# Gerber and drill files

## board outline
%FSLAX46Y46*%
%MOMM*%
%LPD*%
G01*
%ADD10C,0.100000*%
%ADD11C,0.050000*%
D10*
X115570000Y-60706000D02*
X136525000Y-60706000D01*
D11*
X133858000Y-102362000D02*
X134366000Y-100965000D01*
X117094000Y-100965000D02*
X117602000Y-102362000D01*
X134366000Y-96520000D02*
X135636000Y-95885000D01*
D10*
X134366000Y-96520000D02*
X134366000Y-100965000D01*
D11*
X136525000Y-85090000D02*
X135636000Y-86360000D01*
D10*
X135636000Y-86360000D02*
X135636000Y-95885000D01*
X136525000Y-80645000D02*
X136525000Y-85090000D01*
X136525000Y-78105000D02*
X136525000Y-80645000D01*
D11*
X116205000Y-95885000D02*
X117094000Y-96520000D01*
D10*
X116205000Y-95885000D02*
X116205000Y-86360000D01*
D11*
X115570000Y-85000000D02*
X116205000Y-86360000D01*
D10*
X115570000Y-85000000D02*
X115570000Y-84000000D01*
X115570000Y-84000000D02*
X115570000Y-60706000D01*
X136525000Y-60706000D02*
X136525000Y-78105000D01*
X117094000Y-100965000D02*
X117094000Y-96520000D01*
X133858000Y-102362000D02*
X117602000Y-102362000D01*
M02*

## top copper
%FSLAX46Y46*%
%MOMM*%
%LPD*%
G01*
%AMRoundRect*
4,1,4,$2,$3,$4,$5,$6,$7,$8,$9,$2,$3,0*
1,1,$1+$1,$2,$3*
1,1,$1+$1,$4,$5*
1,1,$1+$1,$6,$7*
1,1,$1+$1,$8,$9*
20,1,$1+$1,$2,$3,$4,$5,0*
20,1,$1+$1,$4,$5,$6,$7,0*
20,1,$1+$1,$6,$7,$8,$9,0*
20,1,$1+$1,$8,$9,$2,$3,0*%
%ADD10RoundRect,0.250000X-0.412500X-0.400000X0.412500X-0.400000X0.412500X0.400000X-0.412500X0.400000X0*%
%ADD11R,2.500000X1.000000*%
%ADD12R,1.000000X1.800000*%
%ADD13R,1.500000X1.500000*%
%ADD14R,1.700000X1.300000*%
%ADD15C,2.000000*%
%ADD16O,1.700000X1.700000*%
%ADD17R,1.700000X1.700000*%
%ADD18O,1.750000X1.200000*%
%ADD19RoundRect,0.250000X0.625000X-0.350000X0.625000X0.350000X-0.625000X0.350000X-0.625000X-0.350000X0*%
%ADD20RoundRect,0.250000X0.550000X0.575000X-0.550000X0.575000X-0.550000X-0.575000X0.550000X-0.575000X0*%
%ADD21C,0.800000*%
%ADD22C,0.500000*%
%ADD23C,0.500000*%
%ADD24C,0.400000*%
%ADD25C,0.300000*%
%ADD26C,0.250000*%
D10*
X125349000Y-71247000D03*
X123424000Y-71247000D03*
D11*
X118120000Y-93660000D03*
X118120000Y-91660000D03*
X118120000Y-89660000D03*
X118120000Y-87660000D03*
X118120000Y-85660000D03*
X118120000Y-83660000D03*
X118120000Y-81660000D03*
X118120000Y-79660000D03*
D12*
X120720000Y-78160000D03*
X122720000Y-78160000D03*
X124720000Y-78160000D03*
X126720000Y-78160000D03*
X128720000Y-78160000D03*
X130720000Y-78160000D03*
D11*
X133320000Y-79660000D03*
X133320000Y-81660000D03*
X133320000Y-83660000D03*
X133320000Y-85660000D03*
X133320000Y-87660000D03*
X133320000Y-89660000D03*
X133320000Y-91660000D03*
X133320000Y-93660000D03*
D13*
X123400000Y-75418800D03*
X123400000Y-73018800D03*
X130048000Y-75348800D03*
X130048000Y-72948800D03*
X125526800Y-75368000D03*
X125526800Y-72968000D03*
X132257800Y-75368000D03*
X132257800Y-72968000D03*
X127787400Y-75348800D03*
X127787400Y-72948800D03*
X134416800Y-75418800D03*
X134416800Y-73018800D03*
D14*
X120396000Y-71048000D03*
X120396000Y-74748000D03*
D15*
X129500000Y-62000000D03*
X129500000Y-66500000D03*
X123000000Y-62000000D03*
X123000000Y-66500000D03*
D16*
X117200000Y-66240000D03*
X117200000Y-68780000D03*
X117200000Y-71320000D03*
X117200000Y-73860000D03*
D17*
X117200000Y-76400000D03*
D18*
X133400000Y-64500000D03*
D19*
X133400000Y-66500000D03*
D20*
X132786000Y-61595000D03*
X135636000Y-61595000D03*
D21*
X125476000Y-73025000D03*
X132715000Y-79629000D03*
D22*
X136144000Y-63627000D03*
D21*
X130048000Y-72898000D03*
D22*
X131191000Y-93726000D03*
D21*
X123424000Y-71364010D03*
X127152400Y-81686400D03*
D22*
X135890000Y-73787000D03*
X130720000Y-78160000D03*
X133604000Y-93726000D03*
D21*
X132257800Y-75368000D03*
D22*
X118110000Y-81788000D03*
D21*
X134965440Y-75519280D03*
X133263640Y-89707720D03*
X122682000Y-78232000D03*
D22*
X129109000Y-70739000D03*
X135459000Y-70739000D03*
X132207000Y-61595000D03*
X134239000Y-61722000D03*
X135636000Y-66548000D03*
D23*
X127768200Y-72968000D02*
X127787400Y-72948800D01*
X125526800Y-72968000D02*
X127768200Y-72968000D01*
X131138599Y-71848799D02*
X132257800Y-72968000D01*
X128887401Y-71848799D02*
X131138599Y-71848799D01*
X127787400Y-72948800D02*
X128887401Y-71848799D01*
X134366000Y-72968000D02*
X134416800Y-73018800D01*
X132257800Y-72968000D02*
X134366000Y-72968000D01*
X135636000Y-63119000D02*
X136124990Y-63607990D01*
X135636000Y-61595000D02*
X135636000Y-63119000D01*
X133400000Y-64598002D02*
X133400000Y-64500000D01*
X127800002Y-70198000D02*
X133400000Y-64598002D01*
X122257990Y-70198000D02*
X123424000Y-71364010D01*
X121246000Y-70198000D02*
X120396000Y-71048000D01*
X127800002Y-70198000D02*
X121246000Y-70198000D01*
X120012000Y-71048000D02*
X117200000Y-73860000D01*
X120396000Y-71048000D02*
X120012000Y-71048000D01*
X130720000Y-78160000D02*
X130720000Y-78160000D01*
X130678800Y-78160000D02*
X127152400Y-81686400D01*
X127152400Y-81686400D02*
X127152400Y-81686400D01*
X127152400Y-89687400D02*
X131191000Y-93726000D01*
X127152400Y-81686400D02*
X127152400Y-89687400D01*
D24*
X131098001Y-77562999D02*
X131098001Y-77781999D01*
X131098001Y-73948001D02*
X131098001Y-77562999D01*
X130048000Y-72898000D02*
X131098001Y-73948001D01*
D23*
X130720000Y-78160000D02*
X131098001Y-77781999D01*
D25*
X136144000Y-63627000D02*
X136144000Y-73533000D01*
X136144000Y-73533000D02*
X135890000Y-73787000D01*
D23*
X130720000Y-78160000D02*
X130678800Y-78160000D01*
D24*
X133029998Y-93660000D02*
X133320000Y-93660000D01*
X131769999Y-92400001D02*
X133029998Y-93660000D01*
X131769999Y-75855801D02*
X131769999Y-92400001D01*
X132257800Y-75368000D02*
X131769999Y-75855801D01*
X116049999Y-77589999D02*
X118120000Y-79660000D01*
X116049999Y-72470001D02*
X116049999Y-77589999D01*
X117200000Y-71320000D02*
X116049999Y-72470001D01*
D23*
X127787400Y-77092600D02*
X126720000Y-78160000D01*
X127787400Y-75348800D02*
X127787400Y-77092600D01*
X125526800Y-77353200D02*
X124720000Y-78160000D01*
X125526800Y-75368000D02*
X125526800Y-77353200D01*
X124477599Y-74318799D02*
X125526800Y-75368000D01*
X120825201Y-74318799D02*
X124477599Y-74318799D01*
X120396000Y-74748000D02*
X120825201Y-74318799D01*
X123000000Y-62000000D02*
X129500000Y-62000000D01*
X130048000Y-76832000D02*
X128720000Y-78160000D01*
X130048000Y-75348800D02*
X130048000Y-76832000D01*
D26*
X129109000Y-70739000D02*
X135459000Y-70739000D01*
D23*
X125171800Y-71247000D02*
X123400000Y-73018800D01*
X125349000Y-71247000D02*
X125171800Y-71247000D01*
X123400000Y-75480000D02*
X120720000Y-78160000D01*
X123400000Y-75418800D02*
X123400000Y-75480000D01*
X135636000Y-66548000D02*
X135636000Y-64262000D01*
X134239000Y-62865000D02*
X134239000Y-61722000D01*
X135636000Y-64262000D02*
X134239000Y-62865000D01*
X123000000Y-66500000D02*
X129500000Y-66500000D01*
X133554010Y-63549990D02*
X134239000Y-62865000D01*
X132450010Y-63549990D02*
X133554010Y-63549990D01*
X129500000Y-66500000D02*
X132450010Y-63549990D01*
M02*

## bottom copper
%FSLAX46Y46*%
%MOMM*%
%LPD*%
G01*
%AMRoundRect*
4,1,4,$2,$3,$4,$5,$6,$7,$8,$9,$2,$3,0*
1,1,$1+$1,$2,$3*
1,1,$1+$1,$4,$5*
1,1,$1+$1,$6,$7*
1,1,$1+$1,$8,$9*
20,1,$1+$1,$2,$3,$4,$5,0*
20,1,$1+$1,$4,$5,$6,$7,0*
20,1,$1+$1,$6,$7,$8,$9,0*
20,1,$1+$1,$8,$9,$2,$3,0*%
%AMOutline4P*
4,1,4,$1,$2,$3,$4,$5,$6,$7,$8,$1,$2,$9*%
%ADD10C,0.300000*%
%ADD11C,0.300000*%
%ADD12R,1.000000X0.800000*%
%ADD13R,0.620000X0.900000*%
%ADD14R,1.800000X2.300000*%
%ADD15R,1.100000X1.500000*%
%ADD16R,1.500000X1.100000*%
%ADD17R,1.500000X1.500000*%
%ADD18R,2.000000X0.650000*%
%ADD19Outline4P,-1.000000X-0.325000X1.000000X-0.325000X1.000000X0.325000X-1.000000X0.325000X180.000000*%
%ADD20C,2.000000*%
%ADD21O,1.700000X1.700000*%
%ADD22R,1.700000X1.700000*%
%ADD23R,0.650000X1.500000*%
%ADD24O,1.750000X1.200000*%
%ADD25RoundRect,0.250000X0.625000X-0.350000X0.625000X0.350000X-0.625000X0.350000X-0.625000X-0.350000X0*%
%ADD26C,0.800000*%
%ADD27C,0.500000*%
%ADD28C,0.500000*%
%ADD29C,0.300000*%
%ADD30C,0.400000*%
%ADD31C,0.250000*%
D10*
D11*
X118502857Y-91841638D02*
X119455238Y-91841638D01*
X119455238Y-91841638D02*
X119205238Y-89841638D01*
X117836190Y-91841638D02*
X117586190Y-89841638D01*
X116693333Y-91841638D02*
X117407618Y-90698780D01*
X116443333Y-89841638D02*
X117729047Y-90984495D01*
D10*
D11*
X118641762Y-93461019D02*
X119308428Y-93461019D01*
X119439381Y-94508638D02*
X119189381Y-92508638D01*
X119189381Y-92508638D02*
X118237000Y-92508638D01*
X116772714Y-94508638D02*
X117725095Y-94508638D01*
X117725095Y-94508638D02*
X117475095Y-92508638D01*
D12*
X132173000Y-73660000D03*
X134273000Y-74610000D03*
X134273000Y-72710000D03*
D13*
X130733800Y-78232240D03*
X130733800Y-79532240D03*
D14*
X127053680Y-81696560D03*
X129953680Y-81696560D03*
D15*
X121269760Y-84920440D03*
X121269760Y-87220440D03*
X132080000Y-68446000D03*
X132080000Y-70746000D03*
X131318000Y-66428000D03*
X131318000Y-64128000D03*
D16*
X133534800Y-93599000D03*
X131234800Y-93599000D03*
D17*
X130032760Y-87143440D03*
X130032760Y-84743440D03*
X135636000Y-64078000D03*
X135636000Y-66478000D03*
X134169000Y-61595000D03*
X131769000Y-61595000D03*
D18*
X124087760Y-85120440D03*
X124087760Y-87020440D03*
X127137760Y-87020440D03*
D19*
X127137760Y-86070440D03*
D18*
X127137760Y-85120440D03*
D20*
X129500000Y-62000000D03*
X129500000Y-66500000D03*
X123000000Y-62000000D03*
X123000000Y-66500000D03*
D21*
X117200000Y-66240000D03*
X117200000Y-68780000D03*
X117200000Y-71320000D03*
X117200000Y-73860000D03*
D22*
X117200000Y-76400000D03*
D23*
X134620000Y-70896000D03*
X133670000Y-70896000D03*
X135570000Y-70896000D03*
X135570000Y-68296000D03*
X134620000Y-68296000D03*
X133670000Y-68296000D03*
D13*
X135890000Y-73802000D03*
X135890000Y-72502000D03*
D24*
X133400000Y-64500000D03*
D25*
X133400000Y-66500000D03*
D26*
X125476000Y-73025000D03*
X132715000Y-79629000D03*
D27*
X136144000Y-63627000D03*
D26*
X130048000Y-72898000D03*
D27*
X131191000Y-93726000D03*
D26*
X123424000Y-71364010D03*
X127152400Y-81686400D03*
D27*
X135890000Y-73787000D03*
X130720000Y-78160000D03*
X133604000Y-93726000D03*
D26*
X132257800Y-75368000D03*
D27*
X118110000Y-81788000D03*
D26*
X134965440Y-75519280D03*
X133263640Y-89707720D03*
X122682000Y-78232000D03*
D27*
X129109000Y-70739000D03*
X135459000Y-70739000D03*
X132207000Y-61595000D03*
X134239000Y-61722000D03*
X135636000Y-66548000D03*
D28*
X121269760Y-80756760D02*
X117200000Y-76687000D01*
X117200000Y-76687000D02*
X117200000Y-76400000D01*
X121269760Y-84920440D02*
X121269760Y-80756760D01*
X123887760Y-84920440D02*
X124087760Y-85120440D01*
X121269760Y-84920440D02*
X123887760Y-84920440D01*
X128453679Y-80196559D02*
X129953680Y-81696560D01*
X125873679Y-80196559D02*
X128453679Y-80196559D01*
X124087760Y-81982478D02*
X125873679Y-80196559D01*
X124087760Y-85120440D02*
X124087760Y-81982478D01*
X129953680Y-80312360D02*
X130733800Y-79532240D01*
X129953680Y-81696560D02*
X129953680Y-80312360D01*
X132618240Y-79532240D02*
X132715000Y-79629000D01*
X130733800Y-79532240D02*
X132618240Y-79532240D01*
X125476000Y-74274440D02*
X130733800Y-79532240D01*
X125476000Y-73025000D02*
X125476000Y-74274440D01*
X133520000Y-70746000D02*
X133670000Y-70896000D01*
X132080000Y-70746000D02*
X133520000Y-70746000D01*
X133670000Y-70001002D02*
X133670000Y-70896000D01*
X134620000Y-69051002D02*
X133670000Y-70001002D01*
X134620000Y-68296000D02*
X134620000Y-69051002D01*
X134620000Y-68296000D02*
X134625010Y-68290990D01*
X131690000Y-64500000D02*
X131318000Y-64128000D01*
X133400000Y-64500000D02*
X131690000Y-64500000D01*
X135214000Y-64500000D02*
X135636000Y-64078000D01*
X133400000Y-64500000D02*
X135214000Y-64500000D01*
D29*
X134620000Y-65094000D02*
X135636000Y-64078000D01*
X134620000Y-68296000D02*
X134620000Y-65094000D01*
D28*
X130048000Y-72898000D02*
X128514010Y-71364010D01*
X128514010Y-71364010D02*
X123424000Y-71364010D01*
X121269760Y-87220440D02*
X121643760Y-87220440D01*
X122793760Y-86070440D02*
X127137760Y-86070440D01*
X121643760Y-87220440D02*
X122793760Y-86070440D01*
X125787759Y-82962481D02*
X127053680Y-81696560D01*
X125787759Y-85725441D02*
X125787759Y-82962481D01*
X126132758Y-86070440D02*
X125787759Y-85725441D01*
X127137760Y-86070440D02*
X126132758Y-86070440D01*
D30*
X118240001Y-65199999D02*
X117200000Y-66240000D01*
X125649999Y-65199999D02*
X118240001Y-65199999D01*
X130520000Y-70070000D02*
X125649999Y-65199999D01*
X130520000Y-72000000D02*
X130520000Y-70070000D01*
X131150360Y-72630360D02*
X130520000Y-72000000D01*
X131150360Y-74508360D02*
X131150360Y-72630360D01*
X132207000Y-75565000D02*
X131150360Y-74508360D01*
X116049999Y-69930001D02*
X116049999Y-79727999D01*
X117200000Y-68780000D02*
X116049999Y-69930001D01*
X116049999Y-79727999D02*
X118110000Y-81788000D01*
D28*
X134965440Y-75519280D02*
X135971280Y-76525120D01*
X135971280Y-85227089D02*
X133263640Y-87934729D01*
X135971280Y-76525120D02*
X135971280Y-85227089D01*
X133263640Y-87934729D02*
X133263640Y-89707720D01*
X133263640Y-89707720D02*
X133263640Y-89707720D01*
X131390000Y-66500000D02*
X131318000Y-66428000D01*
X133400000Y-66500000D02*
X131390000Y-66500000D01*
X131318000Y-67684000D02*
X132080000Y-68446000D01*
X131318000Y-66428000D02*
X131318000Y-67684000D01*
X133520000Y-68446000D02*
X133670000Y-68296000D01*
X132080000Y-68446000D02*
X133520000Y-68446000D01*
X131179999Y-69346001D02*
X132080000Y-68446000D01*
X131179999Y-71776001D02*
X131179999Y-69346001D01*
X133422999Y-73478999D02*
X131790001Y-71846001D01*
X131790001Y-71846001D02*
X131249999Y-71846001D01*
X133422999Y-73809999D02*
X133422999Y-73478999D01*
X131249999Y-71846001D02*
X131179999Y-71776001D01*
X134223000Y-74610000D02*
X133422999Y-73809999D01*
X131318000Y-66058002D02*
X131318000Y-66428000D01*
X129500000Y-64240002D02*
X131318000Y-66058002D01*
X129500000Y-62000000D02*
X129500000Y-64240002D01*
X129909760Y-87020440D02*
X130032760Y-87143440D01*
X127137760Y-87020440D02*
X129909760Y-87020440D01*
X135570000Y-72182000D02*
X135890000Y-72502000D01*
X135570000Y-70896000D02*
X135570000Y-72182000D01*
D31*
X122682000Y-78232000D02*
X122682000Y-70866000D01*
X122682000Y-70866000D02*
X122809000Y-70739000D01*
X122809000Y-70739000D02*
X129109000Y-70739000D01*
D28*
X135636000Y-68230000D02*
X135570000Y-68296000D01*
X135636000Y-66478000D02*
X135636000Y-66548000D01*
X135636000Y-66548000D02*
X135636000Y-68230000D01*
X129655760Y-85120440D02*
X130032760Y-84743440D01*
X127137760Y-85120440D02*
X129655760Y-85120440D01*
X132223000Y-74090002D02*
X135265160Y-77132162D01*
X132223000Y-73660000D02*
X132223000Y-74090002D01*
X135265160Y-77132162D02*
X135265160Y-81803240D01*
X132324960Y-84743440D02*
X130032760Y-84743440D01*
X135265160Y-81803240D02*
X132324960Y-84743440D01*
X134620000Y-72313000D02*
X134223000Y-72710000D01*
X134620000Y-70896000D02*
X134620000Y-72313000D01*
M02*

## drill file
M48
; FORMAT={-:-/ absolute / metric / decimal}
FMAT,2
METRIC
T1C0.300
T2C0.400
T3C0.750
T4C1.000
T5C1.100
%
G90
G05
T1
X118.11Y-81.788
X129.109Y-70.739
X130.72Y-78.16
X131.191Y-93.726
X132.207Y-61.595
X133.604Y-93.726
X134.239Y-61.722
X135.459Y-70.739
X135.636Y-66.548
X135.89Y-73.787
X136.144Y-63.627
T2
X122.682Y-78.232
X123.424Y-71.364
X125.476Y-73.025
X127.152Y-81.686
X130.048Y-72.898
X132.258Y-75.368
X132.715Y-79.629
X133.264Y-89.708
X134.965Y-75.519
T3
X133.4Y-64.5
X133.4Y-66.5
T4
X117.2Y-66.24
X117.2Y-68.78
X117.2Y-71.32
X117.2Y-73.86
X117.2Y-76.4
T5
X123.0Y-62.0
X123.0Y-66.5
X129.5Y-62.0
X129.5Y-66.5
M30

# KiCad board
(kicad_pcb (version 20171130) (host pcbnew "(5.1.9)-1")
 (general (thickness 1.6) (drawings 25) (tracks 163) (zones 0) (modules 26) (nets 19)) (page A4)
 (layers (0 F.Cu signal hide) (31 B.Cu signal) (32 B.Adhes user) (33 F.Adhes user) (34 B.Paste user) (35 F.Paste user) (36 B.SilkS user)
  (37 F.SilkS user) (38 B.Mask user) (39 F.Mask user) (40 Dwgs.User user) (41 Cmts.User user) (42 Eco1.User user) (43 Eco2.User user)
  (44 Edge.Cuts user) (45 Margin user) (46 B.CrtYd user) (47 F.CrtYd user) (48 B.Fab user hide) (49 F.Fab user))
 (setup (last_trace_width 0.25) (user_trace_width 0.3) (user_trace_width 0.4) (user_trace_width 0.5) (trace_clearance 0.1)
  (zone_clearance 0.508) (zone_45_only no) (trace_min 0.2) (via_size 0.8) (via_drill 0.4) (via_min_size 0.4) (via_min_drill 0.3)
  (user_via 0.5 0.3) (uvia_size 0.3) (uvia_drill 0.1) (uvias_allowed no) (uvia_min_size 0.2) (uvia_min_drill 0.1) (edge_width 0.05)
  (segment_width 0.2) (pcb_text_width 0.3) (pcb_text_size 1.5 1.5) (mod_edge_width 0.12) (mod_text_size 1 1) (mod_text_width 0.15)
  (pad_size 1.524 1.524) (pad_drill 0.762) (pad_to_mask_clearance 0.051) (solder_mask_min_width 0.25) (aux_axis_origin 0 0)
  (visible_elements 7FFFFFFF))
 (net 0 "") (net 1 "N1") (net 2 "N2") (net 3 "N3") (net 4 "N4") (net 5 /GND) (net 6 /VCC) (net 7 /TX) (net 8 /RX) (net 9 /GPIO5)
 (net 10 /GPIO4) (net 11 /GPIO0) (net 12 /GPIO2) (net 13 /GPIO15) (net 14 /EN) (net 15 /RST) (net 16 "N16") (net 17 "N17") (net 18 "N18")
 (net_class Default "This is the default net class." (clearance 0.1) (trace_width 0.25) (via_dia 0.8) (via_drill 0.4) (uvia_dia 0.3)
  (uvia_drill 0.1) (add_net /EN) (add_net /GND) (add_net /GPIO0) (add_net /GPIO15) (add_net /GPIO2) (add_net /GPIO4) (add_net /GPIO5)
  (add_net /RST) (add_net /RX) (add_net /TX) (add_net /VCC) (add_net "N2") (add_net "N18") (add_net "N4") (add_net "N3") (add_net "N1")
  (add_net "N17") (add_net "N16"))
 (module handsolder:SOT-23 (layer B.Cu) (at 133.223 73.66 180)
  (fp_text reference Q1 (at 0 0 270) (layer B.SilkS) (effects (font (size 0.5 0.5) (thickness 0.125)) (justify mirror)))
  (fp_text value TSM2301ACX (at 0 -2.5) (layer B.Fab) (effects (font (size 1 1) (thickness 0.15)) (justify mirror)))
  (pad 3 smd rect (at 1.05 0 180) (size 1 0.8) (layers B.Cu B.Paste B.Mask) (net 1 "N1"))
  (pad 2 smd rect (at -1.05 -0.95 180) (size 1 0.8) (layers B.Cu B.Paste B.Mask) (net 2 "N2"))
  (pad 1 smd rect (at -1.05 0.95 180) (size 1 0.8) (layers B.Cu B.Paste B.Mask) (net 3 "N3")))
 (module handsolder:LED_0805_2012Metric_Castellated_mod (layer F.Cu) (at 124.3865 71.247)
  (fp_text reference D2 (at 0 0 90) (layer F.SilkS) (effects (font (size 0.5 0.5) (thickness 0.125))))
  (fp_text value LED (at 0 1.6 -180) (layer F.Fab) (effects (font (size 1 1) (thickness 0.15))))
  (pad 2 smd roundrect (at 0.9625 0) (size 1.325 1.3) (layers F.Cu F.Paste F.Mask) (roundrect_rratio 0.1923076923076923) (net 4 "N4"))
  (pad 1 smd roundrect (at -0.9625 0) (size 1.325 1.3) (layers F.Cu F.Paste F.Mask) (roundrect_rratio 0.1923076923076923) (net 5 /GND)))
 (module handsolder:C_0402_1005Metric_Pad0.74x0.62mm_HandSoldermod (layer B.Cu) (at 130.7338 78.88224 90)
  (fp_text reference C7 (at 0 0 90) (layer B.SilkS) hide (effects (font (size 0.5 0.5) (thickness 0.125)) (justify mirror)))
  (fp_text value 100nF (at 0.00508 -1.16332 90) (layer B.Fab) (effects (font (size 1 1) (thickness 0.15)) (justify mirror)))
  (pad 2 smd rect (at 0.65 0 90) (size 0.9 0.62) (layers B.Cu B.Paste B.Mask) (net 5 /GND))
  (pad 1 smd rect (at -0.65 0 90) (size 0.9 0.62) (layers B.Cu B.Paste B.Mask) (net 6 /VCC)))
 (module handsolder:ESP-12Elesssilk (layer F.Cu) (at 125.72 90.16 180)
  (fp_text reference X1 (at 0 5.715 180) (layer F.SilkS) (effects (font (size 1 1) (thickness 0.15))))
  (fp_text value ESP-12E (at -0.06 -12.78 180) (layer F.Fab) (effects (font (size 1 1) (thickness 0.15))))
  (pad 22 smd rect (at 7.6 -3.5 180) (size 2.5 1) (layers F.Cu F.Paste F.Mask))
  (pad 21 smd rect (at 7.6 -1.5 180) (size 2.5 1) (layers F.Cu F.Paste F.Mask))
  (pad 20 smd rect (at 7.6 0.5 180) (size 2.5 1) (layers F.Cu F.Paste F.Mask))
  (pad 19 smd rect (at 7.6 2.5 180) (size 2.5 1) (layers F.Cu F.Paste F.Mask))
  (pad 18 smd rect (at 7.6 4.5 180) (size 2.5 1) (layers F.Cu F.Paste F.Mask))
  (pad 17 smd rect (at 7.6 6.5 180) (size 2.5 1) (layers F.Cu F.Paste F.Mask))
  (pad 16 smd rect (at 7.6 8.5 180) (size 2.5 1) (layers F.Cu F.Paste F.Mask) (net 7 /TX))
  (pad 15 smd rect (at 7.6 10.5 180) (size 2.5 1) (layers F.Cu F.Paste F.Mask) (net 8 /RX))
  (pad 14 smd rect (at 5 12 180) (size 1 1.8) (layers F.Cu F.Paste F.Mask) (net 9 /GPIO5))
  (pad 13 smd rect (at 3 12 180) (size 1 1.8) (layers F.Cu F.Paste F.Mask) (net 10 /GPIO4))
  (pad 12 smd rect (at 1 12 180) (size 1 1.8) (layers F.Cu F.Paste F.Mask) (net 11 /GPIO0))
  (pad 11 smd rect (at -1 12 180) (size 1 1.8) (layers F.Cu F.Paste F.Mask) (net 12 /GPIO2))
  (pad 10 smd rect (at -3 12 180) (size 1 1.8) (layers F.Cu F.Paste F.Mask) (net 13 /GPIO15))
  (pad 9 smd rect (at -5 12 180) (size 1 1.8) (layers F.Cu F.Paste F.Mask) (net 5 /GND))
  (pad 8 smd rect (at -7.6 10.5 180) (size 2.5 1) (layers F.Cu F.Paste F.Mask) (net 6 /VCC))
  (pad 7 smd rect (at -7.6 8.5 180) (size 2.5 1) (layers F.Cu F.Paste F.Mask))
  (pad 6 smd rect (at -7.6 6.5 180) (size 2.5 1) (layers F.Cu F.Paste F.Mask))
  (pad 5 smd rect (at -7.6 4.5 180) (size 2.5 1) (layers F.Cu F.Paste F.Mask))
  (pad 4 smd rect (at -7.6 2.5 180) (size 2.5 1) (layers F.Cu F.Paste F.Mask))
  (pad 3 smd rect (at -7.6 0.5 180) (size 2.5 1) (layers F.Cu F.Paste F.Mask) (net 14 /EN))
  (pad 2 smd rect (at -7.6 -1.5 180) (size 2.5 1) (layers F.Cu F.Paste F.Mask))
  (pad 1 smd rect (at -7.6 -3.5 180) (size 2.5 1) (layers F.Cu F.Paste F.Mask) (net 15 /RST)))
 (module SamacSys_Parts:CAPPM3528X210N (layer B.Cu) (at 128.50368 81.69656 180)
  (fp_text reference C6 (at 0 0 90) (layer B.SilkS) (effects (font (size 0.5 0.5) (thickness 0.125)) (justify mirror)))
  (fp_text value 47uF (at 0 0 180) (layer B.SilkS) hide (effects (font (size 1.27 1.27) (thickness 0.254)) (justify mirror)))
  (pad 2 smd rect (at 1.45 0 180) (size 1.8 2.3) (layers B.Cu B.Paste B.Mask) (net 5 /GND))
  (pad 1 smd rect (at -1.45 0 180) (size 1.8 2.3) (layers B.Cu B.Paste B.Mask) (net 6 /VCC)))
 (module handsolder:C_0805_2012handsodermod (layer B.Cu) (at 121.26976 86.07044 90)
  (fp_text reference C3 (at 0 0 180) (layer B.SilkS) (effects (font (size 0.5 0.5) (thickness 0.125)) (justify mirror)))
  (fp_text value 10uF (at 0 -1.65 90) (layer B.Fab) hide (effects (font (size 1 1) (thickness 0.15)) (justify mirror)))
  (pad 2 smd rect (at 1.15 0 90) (size 1.5 1.1) (layers B.Cu B.Paste B.Mask) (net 6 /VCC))
  (pad 1 smd rect (at -1.15 0 90) (size 1.5 1.1) (layers B.Cu B.Paste B.Mask) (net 5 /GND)))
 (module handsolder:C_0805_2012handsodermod (layer B.Cu) (at 132.08 69.596 90)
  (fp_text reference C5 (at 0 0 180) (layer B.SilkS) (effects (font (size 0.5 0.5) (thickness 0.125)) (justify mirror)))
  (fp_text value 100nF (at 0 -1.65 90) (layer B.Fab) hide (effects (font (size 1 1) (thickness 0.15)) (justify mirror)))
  (pad 2 smd rect (at 1.15 0 90) (size 1.5 1.1) (layers B.Cu B.Paste B.Mask) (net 2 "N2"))
  (pad 1 smd rect (at -1.15 0 90) (size 1.5 1.1) (layers B.Cu B.Paste B.Mask) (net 5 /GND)))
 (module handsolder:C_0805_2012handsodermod (layer B.Cu) (at 131.318 65.278 270)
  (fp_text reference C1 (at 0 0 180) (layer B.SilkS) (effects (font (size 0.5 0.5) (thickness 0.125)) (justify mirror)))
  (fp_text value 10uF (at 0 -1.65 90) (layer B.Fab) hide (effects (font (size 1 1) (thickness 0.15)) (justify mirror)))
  (pad 2 smd rect (at 1.15 0 270) (size 1.5 1.1) (layers B.Cu B.Paste B.Mask) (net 2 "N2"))
  (pad 1 smd rect (at -1.15 0 270) (size 1.5 1.1) (layers B.Cu B.Paste B.Mask) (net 5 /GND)))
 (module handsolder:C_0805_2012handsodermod (layer B.Cu) (at 132.3848 93.599)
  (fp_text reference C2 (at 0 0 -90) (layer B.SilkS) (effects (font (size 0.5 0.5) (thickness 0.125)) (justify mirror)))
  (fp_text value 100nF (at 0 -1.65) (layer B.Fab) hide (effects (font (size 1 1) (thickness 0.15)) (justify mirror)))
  (pad 2 smd rect (at 1.15 0) (size 1.5 1.1) (layers B.Cu B.Paste B.Mask) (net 15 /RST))
  (pad 1 smd rect (at -1.15 0) (size 1.5 1.1) (layers B.Cu B.Paste B.Mask) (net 5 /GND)))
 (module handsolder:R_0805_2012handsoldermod (layer F.Cu) (at 123.4 74.2188 270)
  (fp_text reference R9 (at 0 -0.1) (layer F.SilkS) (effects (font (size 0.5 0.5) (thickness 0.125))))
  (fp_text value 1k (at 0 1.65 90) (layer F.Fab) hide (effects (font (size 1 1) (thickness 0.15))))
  (pad 2 smd rect (at 1.2 0 270) (size 1.5 1.5) (layers F.Cu F.Paste F.Mask) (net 9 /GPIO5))
  (pad 1 smd rect (at -1.2 0 270) (size 1.5 1.5) (layers F.Cu F.Paste F.Mask) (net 4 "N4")))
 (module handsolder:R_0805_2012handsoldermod (layer B.Cu) (at 130.03276 85.94344 270)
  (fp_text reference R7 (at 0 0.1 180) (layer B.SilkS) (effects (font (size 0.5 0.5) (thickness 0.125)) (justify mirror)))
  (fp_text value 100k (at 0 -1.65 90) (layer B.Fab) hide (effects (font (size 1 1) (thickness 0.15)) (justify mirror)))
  (pad 2 smd rect (at 1.2 0 270) (size 1.5 1.5) (layers B.Cu B.Paste B.Mask) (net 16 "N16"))
  (pad 1 smd rect (at -1.2 0 270) (size 1.5 1.5) (layers B.Cu B.Paste B.Mask) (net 1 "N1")))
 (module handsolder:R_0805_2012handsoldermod (layer B.Cu) (at 135.636 65.278 90)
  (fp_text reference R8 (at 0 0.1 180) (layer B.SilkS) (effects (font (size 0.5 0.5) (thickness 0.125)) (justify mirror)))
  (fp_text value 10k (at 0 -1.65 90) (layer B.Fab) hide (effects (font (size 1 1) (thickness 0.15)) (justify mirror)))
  (pad 2 smd rect (at 1.2 0 90) (size 1.5 1.5) (layers B.Cu B.Paste B.Mask) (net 5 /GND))
  (pad 1 smd rect (at -1.2 0 90) (size 1.5 1.5) (layers B.Cu B.Paste B.Mask) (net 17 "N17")))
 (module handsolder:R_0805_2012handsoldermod (layer B.Cu) (at 132.969 61.595)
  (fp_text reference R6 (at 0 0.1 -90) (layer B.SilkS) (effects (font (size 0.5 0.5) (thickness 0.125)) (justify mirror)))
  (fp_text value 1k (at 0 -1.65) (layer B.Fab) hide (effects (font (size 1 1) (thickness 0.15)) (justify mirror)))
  (pad 2 smd rect (at 1.2 0) (size 1.5 1.5) (layers B.Cu B.Paste B.Mask) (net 17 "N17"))
  (pad 1 smd rect (at -1.2 0) (size 1.5 1.5) (layers B.Cu B.Paste B.Mask) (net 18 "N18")))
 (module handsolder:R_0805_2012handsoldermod (layer F.Cu) (at 130.048 74.1488 270)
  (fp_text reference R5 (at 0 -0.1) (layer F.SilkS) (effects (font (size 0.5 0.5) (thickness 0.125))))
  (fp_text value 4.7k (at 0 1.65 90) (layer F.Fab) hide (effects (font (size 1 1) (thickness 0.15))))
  (pad 2 smd rect (at 1.2 0 270) (size 1.5 1.5) (layers F.Cu F.Paste F.Mask) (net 13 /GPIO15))
  (pad 1 smd rect (at -1.2 0 270) (size 1.5 1.5) (layers F.Cu F.Paste F.Mask) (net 5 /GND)))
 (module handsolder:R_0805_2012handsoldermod (layer F.Cu) (at 125.5268 74.168 270)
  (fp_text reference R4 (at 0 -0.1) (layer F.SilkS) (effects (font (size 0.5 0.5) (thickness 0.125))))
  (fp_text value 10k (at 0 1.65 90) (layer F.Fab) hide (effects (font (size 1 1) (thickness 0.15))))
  (pad 2 smd rect (at 1.2 0 270) (size 1.5 1.5) (layers F.Cu F.Paste F.Mask) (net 11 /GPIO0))
  (pad 1 smd rect (at -1.2 0 270) (size 1.5 1.5) (layers F.Cu F.Paste F.Mask) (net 6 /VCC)))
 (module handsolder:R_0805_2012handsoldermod (layer F.Cu) (at 132.2578 74.168 270)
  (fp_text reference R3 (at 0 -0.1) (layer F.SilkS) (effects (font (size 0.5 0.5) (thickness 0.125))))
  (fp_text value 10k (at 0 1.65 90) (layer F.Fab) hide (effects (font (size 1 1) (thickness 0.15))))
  (pad 2 smd rect (at 1.2 0 270) (size 1.5 1.5) (layers F.Cu F.Paste F.Mask) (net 15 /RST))
  (pad 1 smd rect (at -1.2 0 270) (size 1.5 1.5) (layers F.Cu F.Paste F.Mask) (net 6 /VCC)))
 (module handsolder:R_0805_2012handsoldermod (layer F.Cu) (at 127.7874 74.1488 270)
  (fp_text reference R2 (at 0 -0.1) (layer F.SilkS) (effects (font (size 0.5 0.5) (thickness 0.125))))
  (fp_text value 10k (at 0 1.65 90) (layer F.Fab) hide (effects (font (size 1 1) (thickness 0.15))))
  (pad 2 smd rect (at 1.2 0 270) (size 1.5 1.5) (layers F.Cu F.Paste F.Mask) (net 12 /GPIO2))
  (pad 1 smd rect (at -1.2 0 270) (size 1.5 1.5) (layers F.Cu F.Paste F.Mask) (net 6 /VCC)))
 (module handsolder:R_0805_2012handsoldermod (layer F.Cu) (at 134.4168 74.2188 270)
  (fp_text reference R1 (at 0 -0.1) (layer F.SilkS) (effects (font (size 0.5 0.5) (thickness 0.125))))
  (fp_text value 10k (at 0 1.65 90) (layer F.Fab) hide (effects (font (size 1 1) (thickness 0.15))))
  (pad 2 smd rect (at 1.2 0 270) (size 1.5 1.5) (layers F.Cu F.Paste F.Mask) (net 14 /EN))
  (pad 1 smd rect (at -1.2 0 270) (size 1.5 1.5) (layers F.Cu F.Paste F.Mask) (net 6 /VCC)))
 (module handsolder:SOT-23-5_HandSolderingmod (layer B.Cu) (at 125.58776 86.07044 180)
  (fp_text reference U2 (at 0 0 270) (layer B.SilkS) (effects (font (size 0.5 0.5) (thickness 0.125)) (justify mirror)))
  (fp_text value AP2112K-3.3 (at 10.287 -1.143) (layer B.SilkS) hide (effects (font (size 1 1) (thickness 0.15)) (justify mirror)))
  (pad 5 smd rect (at 1.5 0.95 180) (size 2 0.65) (layers B.Cu B.Paste B.Mask) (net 6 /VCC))
  (pad 4 smd rect (at 1.5 -0.95 180) (size 2 0.65) (layers B.Cu B.Paste B.Mask))
  (pad 3 smd rect (at -1.55 -0.95 180) (size 2 0.65) (layers B.Cu B.Paste B.Mask) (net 16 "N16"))
  (pad 2 smd trapezoid (at -1.55 0 180) (size 2 0.65) (layers B.Cu B.Paste B.Mask) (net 5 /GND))
  (pad 1 smd rect (at -1.55 0.95 180) (size 2 0.65) (layers B.Cu B.Paste B.Mask) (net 1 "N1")))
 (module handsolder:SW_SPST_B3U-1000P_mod (layer F.Cu) (at 120.396 72.898 90)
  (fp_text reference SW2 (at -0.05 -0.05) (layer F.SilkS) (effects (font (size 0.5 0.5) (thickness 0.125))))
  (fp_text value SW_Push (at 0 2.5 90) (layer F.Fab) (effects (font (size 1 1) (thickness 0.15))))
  (pad 2 smd rect (at 1.85 0 90) (size 1.3 1.7) (layers F.Cu F.Paste F.Mask) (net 5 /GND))
  (pad 1 smd rect (at -1.85 0 90) (size 1.3 1.7) (layers F.Cu F.Paste F.Mask) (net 11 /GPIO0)))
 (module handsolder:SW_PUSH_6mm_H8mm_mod (layer F.Cu) (at 123 62)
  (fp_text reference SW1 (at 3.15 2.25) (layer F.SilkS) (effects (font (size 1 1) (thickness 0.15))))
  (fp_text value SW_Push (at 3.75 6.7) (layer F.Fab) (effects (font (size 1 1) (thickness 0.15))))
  (pad 1 thru_hole circle (at 6.5 0 90) (size 2 2) (drill 1.1) (layers *.Cu *.Mask) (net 2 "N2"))
  (pad 2 thru_hole circle (at 6.5 4.5 90) (size 2 2) (drill 1.1) (layers *.Cu *.Mask) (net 17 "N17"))
  (pad 1 thru_hole circle (at 0 0 90) (size 2 2) (drill 1.1) (layers *.Cu *.Mask) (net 2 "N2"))
  (pad 2 thru_hole circle (at 0 4.5 90) (size 2 2) (drill 1.1) (layers *.Cu *.Mask) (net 17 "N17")))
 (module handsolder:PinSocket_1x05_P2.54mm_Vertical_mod (layer F.Cu) (at 117.2 76.4 180)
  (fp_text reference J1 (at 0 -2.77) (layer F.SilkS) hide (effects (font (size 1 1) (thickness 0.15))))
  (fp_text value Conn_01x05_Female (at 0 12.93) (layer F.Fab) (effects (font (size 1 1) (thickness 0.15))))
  (pad 5 thru_hole oval (at 0 10.16 180) (size 1.7 1.7) (drill 1) (layers *.Cu *.Mask) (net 15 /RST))
  (pad 4 thru_hole oval (at 0 7.62 180) (size 1.7 1.7) (drill 1) (layers *.Cu *.Mask) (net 7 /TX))
  (pad 3 thru_hole oval (at 0 5.08 180) (size 1.7 1.7) (drill 1) (layers *.Cu *.Mask) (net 8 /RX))
  (pad 2 thru_hole oval (at 0 2.54 180) (size 1.7 1.7) (drill 1) (layers *.Cu *.Mask) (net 5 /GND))
  (pad 1 thru_hole rect (at 0 0 180) (size 1.7 1.7) (drill 1) (layers *.Cu *.Mask) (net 6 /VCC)))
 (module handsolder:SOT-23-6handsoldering (layer B.Cu) (at 134.62 69.596 270)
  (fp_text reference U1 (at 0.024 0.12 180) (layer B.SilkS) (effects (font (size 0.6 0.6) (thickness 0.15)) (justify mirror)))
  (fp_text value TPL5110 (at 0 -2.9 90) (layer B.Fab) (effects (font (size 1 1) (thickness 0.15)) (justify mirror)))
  (pad 5 smd rect (at 1.3 0 270) (size 1.5 0.65) (layers B.Cu B.Paste B.Mask) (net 3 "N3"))
  (pad 6 smd rect (at 1.3 0.95 270) (size 1.5 0.65) (layers B.Cu B.Paste B.Mask) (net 5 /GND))
  (pad 4 smd rect (at 1.3 -0.95 270) (size 1.5 0.65) (layers B.Cu B.Paste B.Mask) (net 10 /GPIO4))
  (pad 3 smd rect (at -1.3 -0.95 270) (size 1.5 0.65) (layers B.Cu B.Paste B.Mask) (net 17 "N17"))
  (pad 2 smd rect (at -1.3 0 270) (size 1.5 0.65) (layers B.Cu B.Paste B.Mask) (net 5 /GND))
  (pad 1 smd rect (at -1.3 0.95 270) (size 1.5 0.65) (layers B.Cu B.Paste B.Mask) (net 2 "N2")))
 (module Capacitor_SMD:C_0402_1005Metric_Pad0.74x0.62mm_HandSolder (layer B.Cu) (at 135.89 73.152 270)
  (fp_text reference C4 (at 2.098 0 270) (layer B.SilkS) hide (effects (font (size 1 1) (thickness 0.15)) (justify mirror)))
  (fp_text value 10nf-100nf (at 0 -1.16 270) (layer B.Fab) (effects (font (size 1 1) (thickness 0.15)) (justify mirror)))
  (pad 2 smd rect (at 0.65 0 270) (size 0.9 0.62) (layers B.Cu B.Paste B.Mask) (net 5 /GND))
  (pad 1 smd rect (at -0.65 0 270) (size 0.9 0.62) (layers B.Cu B.Paste B.Mask) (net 10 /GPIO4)))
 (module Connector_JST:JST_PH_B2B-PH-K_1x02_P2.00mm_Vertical (layer F.Cu) (at 133.4 66.5 90)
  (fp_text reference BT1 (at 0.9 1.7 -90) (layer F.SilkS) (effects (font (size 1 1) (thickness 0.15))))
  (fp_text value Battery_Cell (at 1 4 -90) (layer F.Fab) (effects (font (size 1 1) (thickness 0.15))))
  (pad 2 thru_hole oval (at 2 0 90) (size 1.2 1.75) (drill 0.75) (layers *.Cu *.Mask) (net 5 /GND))
  (pad 1 thru_hole roundrect (at 0 0 90) (size 1.2 1.75) (drill 0.75) (layers *.Cu *.Mask) (roundrect_rratio 0.208333) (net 2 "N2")))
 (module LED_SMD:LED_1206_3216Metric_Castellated (layer F.Cu) (at 134.211 61.595 180)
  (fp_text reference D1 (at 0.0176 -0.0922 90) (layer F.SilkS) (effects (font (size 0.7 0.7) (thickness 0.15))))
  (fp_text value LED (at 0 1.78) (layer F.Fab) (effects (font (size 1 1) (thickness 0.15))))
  (pad 2 smd roundrect (at 1.425 0 180) (size 1.6 1.65) (layers F.Cu F.Paste F.Mask) (roundrect_rratio 0.15625) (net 18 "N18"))
  (pad 1 smd roundrect (at -1.425 0 180) (size 1.6 1.65) (layers F.Cu F.Paste F.Mask) (roundrect_rratio 0.15625) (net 5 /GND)))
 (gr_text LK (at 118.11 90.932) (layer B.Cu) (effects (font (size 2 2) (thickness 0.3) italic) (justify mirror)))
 (gr_line (start 115.57 60.706) (end 136.525 60.706) (layer Edge.Cuts) (width 0.1))
 (gr_line (start 133.858 102.362) (end 134.366 100.965) (layer Edge.Cuts) (width 0.05))
 (gr_line (start 117.094 100.965) (end 117.602 102.362) (layer Edge.Cuts) (width 0.05))
 (gr_line (start 134.366 96.52) (end 135.636 95.885) (layer Edge.Cuts) (width 0.05))
 (gr_line (start 134.366 96.52) (end 134.366 100.965) (layer Edge.Cuts) (width 0.1))
 (gr_line (start 136.525 85.09) (end 135.636 86.36) (layer Edge.Cuts) (width 0.05))
 (gr_line (start 135.636 86.36) (end 135.636 95.885) (layer Edge.Cuts) (width 0.1))
 (gr_line (start 136.525 80.645) (end 136.525 85.09) (layer Edge.Cuts) (width 0.1))
 (gr_line (start 136.525 78.105) (end 136.525 80.645) (layer Edge.Cuts) (width 0.1))
 (gr_line (start 116.205 95.885) (end 117.094 96.52) (layer Edge.Cuts) (width 0.05))
 (gr_line (start 116.205 95.885) (end 116.205 86.36) (layer Edge.Cuts) (width 0.1))
 (gr_line (start 115.57 85) (end 116.205 86.36) (layer Edge.Cuts) (width 0.05))
 (gr_line (start 115.57 85) (end 115.57 84) (layer Edge.Cuts) (width 0.1))
 (gr_line (start 115.57 84) (end 115.57 60.706) (layer Edge.Cuts) (width 0.1))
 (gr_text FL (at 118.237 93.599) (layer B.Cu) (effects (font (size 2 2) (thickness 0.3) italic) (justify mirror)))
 (gr_line (start 136.525 60.706) (end 136.525 78.105) (layer Edge.Cuts) (width 0.1))
 (gr_line (start 117.094 100.965) (end 117.094 96.52) (layer Edge.Cuts) (width 0.1))
 (gr_line (start 133.858 102.362) (end 117.602 102.362) (layer Edge.Cuts) (width 0.1))
 (via (at 125.476 73.025) (size 0.8) (drill 0.4) (layers F.Cu B.Cu) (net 6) (status 30))
 (via (at 132.715 79.629) (size 0.8) (drill 0.4) (layers F.Cu B.Cu) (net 6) (status 30))
 (segment (start 127.7682 72.968) (end 127.7874 72.9488) (width 0.5) (layer F.Cu) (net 6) (status 30))
 (segment (start 125.5268 72.968) (end 127.7682 72.968) (width 0.5) (layer F.Cu) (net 6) (status 30))
 (segment (start 131.138599 71.848799) (end 132.2578 72.968) (width 0.5) (layer F.Cu) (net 6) (status 20))
 (segment (start 128.887401 71.848799) (end 131.138599 71.848799) (width 0.5) (layer F.Cu) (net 6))
 (segment (start 127.7874 72.9488) (end 128.887401 71.848799) (width 0.5) (layer F.Cu) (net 6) (status 10))
 (segment (start 134.366 72.968) (end 134.4168 73.0188) (width 0.5) (layer F.Cu) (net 6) (status 30))
 (segment (start 132.2578 72.968) (end 134.366 72.968) (width 0.5) (layer F.Cu) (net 6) (status 30))
 (segment (start 121.26976 80.75676) (end 117.2 76.687) (width 0.5) (layer B.Cu) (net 6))
 (segment (start 117.2 76.687) (end 117.2 76.4) (width 0.5) (layer B.Cu) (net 6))
 (segment (start 121.26976 84.92044) (end 121.26976 80.75676) (width 0.5) (layer B.Cu) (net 6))
 (segment (start 123.88776 84.92044) (end 124.08776 85.12044) (width 0.5) (layer B.Cu) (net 6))
 (segment (start 121.26976 84.92044) (end 123.88776 84.92044) (width 0.5) (layer B.Cu) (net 6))
 (segment (start 128.453679 80.196559) (end 129.95368 81.69656) (width 0.5) (layer B.Cu) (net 6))
 (segment (start 125.873679 80.196559) (end 128.453679 80.196559) (width 0.5) (layer B.Cu) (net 6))
 (segment (start 124.08776 81.982478) (end 125.873679 80.196559) (width 0.5) (layer B.Cu) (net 6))
 (segment (start 124.08776 85.12044) (end 124.08776 81.982478) (width 0.5) (layer B.Cu) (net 6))
 (segment (start 129.95368 80.31236) (end 130.7338 79.53224) (width 0.5) (layer B.Cu) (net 6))
 (segment (start 129.95368 81.69656) (end 129.95368 80.31236) (width 0.5) (layer B.Cu) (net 6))
 (segment (start 132.61824 79.53224) (end 132.715 79.629) (width 0.5) (layer B.Cu) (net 6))
 (segment (start 130.7338 79.53224) (end 132.61824 79.53224) (width 0.5) (layer B.Cu) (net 6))
 (segment (start 125.476 74.27444) (end 130.7338 79.53224) (width 0.5) (layer B.Cu) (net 6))
 (segment (start 125.476 73.025) (end 125.476 74.27444) (width 0.5) (layer B.Cu) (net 6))
 (via (at 136.144 63.627) (size 0.5) (drill 0.3) (layers F.Cu B.Cu) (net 5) (status 30))
 (segment (start 133.52 70.746) (end 133.67 70.896) (width 0.5) (layer B.Cu) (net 5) (status 30))
 (segment (start 132.08 70.746) (end 133.52 70.746) (width 0.5) (layer B.Cu) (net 5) (status 30))
 (segment (start 133.67 70.001002) (end 133.67 70.896) (width 0.5) (layer B.Cu) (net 5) (status 20))
 (segment (start 134.62 69.051002) (end 133.67 70.001002) (width 0.5) (layer B.Cu) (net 5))
 (segment (start 134.62 68.296) (end 134.62 69.051002) (width 0.5) (layer B.Cu) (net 5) (status 10))
 (segment (start 134.62 68.296) (end 134.62501 68.29099) (width 0.5) (layer B.Cu) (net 5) (status 30))
 (segment (start 131.69 64.5) (end 131.318 64.128) (width 0.5) (layer B.Cu) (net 5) (status 30))
 (segment (start 133.4 64.5) (end 131.69 64.5) (width 0.5) (layer B.Cu) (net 5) (status 30))
 (segment (start 135.214 64.5) (end 135.636 64.078) (width 0.5) (layer B.Cu) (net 5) (status 30))
 (segment (start 133.4 64.5) (end 135.214 64.5) (width 0.5) (layer B.Cu) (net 5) (status 30))
 (segment (start 134.62 65.094) (end 135.636 64.078) (width 0.3) (layer B.Cu) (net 5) (status 20))
 (segment (start 134.62 68.296) (end 134.62 65.094) (width 0.3) (layer B.Cu) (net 5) (status 10))
 (segment (start 135.636 63.119) (end 136.12499 63.60799) (width 0.5) (layer F.Cu) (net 5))
 (segment (start 135.636 61.595) (end 135.636 63.119) (width 0.5) (layer F.Cu) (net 5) (status 10))
 (via (at 130.048 72.898) (size 0.8) (drill 0.4) (layers F.Cu B.Cu) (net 5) (status 30))
 (segment (start 133.4 64.598002) (end 133.4 64.5) (width 0.5) (layer F.Cu) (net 5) (status 30))
 (segment (start 127.800002 70.198) (end 133.4 64.598002) (width 0.5) (layer F.Cu) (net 5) (status 20))
 (via (at 131.191 93.726) (size 0.5) (drill 0.3) (layers F.Cu B.Cu) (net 5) (status 30))
 (via (at 123.424 71.36401) (size 0.8) (drill 0.4) (layers F.Cu B.Cu) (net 5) (status 30))
 (segment (start 122.25799 70.198) (end 123.424 71.36401) (width 0.5) (layer F.Cu) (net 5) (status 20))
 (segment (start 130.048 72.898) (end 128.51401 71.36401) (width 0.5) (layer B.Cu) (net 5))
 (segment (start 128.51401 71.36401) (end 123.424 71.36401) (width 0.5) (layer B.Cu) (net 5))
 (segment (start 121.246 70.198) (end 120.396 71.048) (width 0.5) (layer F.Cu) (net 5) (status 20))
 (segment (start 127.800002 70.198) (end 121.246 70.198) (width 0.5) (layer F.Cu) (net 5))
 (segment (start 120.012 71.048) (end 117.2 73.86) (width 0.5) (layer F.Cu) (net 5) (status 30))
 (segment (start 120.396 71.048) (end 120.012 71.048) (width 0.5) (layer F.Cu) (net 5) (status 30))
 (segment (start 121.26976 87.22044) (end 121.64376 87.22044) (width 0.5) (layer B.Cu) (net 5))
 (segment (start 122.79376 86.07044) (end 127.13776 86.07044) (width 0.5) (layer B.Cu) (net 5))
 (segment (start 121.64376 87.22044) (end 122.79376 86.07044) (width 0.5) (layer B.Cu) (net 5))
 (segment (start 125.787759 82.962481) (end 127.05368 81.69656) (width 0.5) (layer B.Cu) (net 5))
 (segment (start 125.787759 85.725441) (end 125.787759 82.962481) (width 0.5) (layer B.Cu) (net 5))
 (segment (start 126.132758 86.07044) (end 125.787759 85.725441) (width 0.5) (layer B.Cu) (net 5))
 (segment (start 127.13776 86.07044) (end 126.132758 86.07044) (width 0.5) (layer B.Cu) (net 5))
 (segment (start 130.72 78.16) (end 130.72 78.16) (width 0.5) (layer F.Cu) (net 5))
 (segment (start 130.6788 78.16) (end 127.1524 81.6864) (width 0.5) (layer F.Cu) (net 5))
 (segment (start 127.1524 81.6864) (end 127.1524 81.6864) (width 0.5) (layer F.Cu) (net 5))
 (via (at 127.1524 81.6864) (size 0.8) (drill 0.4) (layers F.Cu B.Cu) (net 5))
 (segment (start 127.1524 89.6874) (end 131.191 93.726) (width 0.5) (layer F.Cu) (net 5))
 (segment (start 127.1524 81.6864) (end 127.1524 89.6874) (width 0.5) (layer F.Cu) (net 5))
 (segment (start 131.098001 77.562999) (end 131.098001 77.781999) (width 0.4) (layer F.Cu) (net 5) (status 30))
 (segment (start 131.098001 73.948001) (end 131.098001 77.562999) (width 0.4) (layer F.Cu) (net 5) (status 20))
 (segment (start 130.048 72.898) (end 131.098001 73.948001) (width 0.4) (layer F.Cu) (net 5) (status 10))
 (segment (start 130.72 78.16) (end 131.098001 77.781999) (width 0.5) (layer F.Cu) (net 5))
 (via (at 135.89 73.787) (size 0.5) (drill 0.3) (layers F.Cu B.Cu) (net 5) (status 30))
 (segment (start 136.144 63.627) (end 136.144 73.533) (width 0.3) (layer F.Cu) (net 5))
 (segment (start 136.144 73.533) (end 135.89 73.787) (width 0.3) (layer F.Cu) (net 5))
 (segment (start 130.72 78.16) (end 130.6788 78.16) (width 0.5) (layer F.Cu) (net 5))
 (via (at 130.72 78.16) (size 0.5) (drill 0.3) (layers F.Cu B.Cu) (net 5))
 (via (at 133.604 93.726) (size 0.5) (drill 0.3) (layers F.Cu B.Cu) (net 15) (status 30))
 (segment (start 133.029998 93.66) (end 133.32 93.66) (width 0.4) (layer F.Cu) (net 15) (status 30))
 (segment (start 131.769999 92.400001) (end 133.029998 93.66) (width 0.4) (layer F.Cu) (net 15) (status 20))
 (segment (start 131.769999 75.855801) (end 131.769999 92.400001) (width 0.4) (layer F.Cu) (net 15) (status 10))
 (segment (start 132.2578 75.368) (end 131.769999 75.855801) (width 0.4) (layer F.Cu) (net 15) (status 30))
 (via (at 132.2578 75.368) (size 0.8) (drill 0.4) (layers F.Cu B.Cu) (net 15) (status 30))
 (segment (start 118.240001 65.199999) (end 117.2 66.24) (width 0.4) (layer B.Cu) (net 15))
 (segment (start 125.649999 65.199999) (end 118.240001 65.199999) (width 0.4) (layer B.Cu) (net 15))
 (segment (start 130.52 70.07) (end 125.649999 65.199999) (width 0.4) (layer B.Cu) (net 15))
 (segment (start 130.52 72) (end 130.52 70.07) (width 0.4) (layer B.Cu) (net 15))
 (segment (start 131.15036 72.63036) (end 130.52 72) (width 0.4) (layer B.Cu) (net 15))
 (segment (start 131.15036 74.50836) (end 131.15036 72.63036) (width 0.4) (layer B.Cu) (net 15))
 (segment (start 132.207 75.565) (end 131.15036 74.50836) (width 0.4) (layer B.Cu) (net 15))
 (segment (start 116.049999 77.589999) (end 118.12 79.66) (width 0.4) (layer F.Cu) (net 8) (status 20))
 (segment (start 116.049999 72.470001) (end 116.049999 77.589999) (width 0.4) (layer F.Cu) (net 8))
 (segment (start 117.2 71.32) (end 116.049999 72.470001) (width 0.4) (layer F.Cu) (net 8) (status 10))
 (segment (start 116.049999 69.930001) (end 116.049999 79.727999) (width 0.4) (layer B.Cu) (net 7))
 (segment (start 117.2 68.78) (end 116.049999 69.930001) (width 0.4) (layer B.Cu) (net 7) (status 10))
 (segment (start 116.049999 79.727999) (end 118.11 81.788) (width 0.4) (layer B.Cu) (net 7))
 (via (at 118.11 81.788) (size 0.5) (drill 0.3) (layers F.Cu B.Cu) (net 7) (status 30))
 (via (at 134.96544 75.51928) (size 0.8) (drill 0.4) (layers F.Cu B.Cu) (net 14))
 (segment (start 134.96544 75.51928) (end 135.97128 76.52512) (width 0.5) (layer B.Cu) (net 14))
 (segment (start 135.97128 85.227089) (end 133.26364 87.934729) (width 0.5) (layer B.Cu) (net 14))
 (segment (start 135.97128 76.52512) (end 135.97128 85.227089) (width 0.5) (layer B.Cu) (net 14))
 (segment (start 133.26364 87.934729) (end 133.26364 89.70772) (width 0.5) (layer B.Cu) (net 14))
 (segment (start 133.26364 89.70772) (end 133.26364 89.70772) (width 0.5) (layer B.Cu) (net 14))
 (via (at 133.26364 89.70772) (size 0.8) (drill 0.4) (layers F.Cu B.Cu) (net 14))
 (segment (start 127.7874 77.0926) (end 126.72 78.16) (width 0.5) (layer F.Cu) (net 12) (status 20))
 (segment (start 127.7874 75.3488) (end 127.7874 77.0926) (width 0.5) (layer F.Cu) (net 12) (status 10))
 (segment (start 125.5268 77.3532) (end 124.72 78.16) (width 0.5) (layer F.Cu) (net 11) (status 20))
 (segment (start 125.5268 75.368) (end 125.5268 77.3532) (width 0.5) (layer F.Cu) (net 11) (status 10))
 (segment (start 124.477599 74.318799) (end 125.5268 75.368) (width 0.5) (layer F.Cu) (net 11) (status 20))
 (segment (start 120.825201 74.318799) (end 124.477599 74.318799) (width 0.5) (layer F.Cu) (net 11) (status 10))
 (segment (start 120.396 74.748) (end 120.825201 74.318799) (width 0.5) (layer F.Cu) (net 11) (status 30))
 (segment (start 131.39 66.5) (end 131.318 66.428) (width 0.5) (layer B.Cu) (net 2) (status 30))
 (segment (start 133.4 66.5) (end 131.39 66.5) (width 0.5) (layer B.Cu) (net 2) (status 30))
 (segment (start 131.318 67.684) (end 132.08 68.446) (width 0.5) (layer B.Cu) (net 2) (status 20))
 (segment (start 131.318 66.428) (end 131.318 67.684) (width 0.5) (layer B.Cu) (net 2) (status 10))
 (segment (start 133.52 68.446) (end 133.67 68.296) (width 0.5) (layer B.Cu) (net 2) (status 30))
 (segment (start 132.08 68.446) (end 133.52 68.446) (width 0.5) (layer B.Cu) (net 2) (status 30))
 (segment (start 131.179999 69.346001) (end 132.08 68.446) (width 0.5) (layer B.Cu) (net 2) (status 20))
 (segment (start 131.179999 71.776001) (end 131.179999 69.346001) (width 0.5) (layer B.Cu) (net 2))
 (segment (start 133.422999 73.478999) (end 131.790001 71.846001) (width 0.5) (layer B.Cu) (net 2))
 (segment (start 131.790001 71.846001) (end 131.249999 71.846001) (width 0.5) (layer B.Cu) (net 2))
 (segment (start 133.422999 73.809999) (end 133.422999 73.478999) (width 0.5) (layer B.Cu) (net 2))
 (segment (start 131.249999 71.846001) (end 131.179999 71.776001) (width 0.5) (layer B.Cu) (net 2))
 (segment (start 134.223 74.61) (end 133.422999 73.809999) (width 0.5) (layer B.Cu) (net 2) (status 10))
 (segment (start 123 62) (end 129.5 62) (width 0.5) (layer F.Cu) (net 2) (status 30))
 (segment (start 131.318 66.058002) (end 131.318 66.428) (width 0.5) (layer B.Cu) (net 2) (status 30))
 (segment (start 129.5 64.240002) (end 131.318 66.058002) (width 0.5) (layer B.Cu) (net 2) (status 20))
 (segment (start 129.5 62) (end 129.5 64.240002) (width 0.5) (layer B.Cu) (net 2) (status 10))
 (segment (start 130.048 76.832) (end 128.72 78.16) (width 0.5) (layer F.Cu) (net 13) (status 20))
 (segment (start 130.048 75.3488) (end 130.048 76.832) (width 0.5) (layer F.Cu) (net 13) (status 10))
 (segment (start 129.90976 87.02044) (end 130.03276 87.14344) (width 0.5) (layer B.Cu) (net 16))
 (segment (start 127.13776 87.02044) (end 129.90976 87.02044) (width 0.5) (layer B.Cu) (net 16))
 (via (at 122.682 78.232) (size 0.8) (drill 0.4) (layers F.Cu B.Cu) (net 10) (status 30))
 (segment (start 135.57 72.182) (end 135.89 72.502) (width 0.5) (layer B.Cu) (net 10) (status 20))
 (segment (start 135.57 70.896) (end 135.57 72.182) (width 0.5) (layer B.Cu) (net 10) (status 10))
 (segment (start 122.682 78.232) (end 122.682 70.866) (width 0.25) (layer B.Cu) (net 10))
 (segment (start 122.682 70.866) (end 122.809 70.739) (width 0.25) (layer B.Cu) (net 10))
 (segment (start 122.809 70.739) (end 129.109 70.739) (width 0.25) (layer B.Cu) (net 10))
 (via (at 129.109 70.739) (size 0.5) (drill 0.3) (layers F.Cu B.Cu) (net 10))
 (segment (start 129.109 70.739) (end 135.459 70.739) (width 0.25) (layer F.Cu) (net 10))
 (via (at 135.459 70.739) (size 0.5) (drill 0.3) (layers F.Cu B.Cu) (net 10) (status 30))
 (segment (start 125.1718 71.247) (end 123.4 73.0188) (width 0.5) (layer F.Cu) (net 4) (status 30))
 (segment (start 125.349 71.247) (end 125.1718 71.247) (width 0.5) (layer F.Cu) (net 4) (status 30))
 (segment (start 123.4 75.48) (end 120.72 78.16) (width 0.5) (layer F.Cu) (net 9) (status 30))
 (segment (start 123.4 75.4188) (end 123.4 75.48) (width 0.5) (layer F.Cu) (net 9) (status 30))
 (via (at 132.207 61.595) (size 0.5) (drill 0.3) (layers F.Cu B.Cu) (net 18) (status 30))
 (via (at 134.239 61.722) (size 0.5) (drill 0.3) (layers F.Cu B.Cu) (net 17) (status 30))
 (segment (start 135.636 68.23) (end 135.57 68.296) (width 0.5) (layer B.Cu) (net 17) (status 30))
 (segment (start 135.636 66.478) (end 135.636 66.548) (width 0.5) (layer B.Cu) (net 17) (status 30))
 (segment (start 135.636 66.548) (end 135.636 68.23) (width 0.5) (layer B.Cu) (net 17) (status 30))
 (via (at 135.636 66.548) (size 0.5) (drill 0.3) (layers F.Cu B.Cu) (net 17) (status 30))
 (segment (start 135.636 66.548) (end 135.636 64.262) (width 0.5) (layer F.Cu) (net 17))
 (segment (start 134.239 62.865) (end 134.239 61.722) (width 0.5) (layer F.Cu) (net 17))
 (segment (start 135.636 64.262) (end 134.239 62.865) (width 0.5) (layer F.Cu) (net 17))
 (segment (start 123 66.5) (end 129.5 66.5) (width 0.5) (layer F.Cu) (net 17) (status 30))
 (segment (start 133.55401 63.54999) (end 134.239 62.865) (width 0.5) (layer F.Cu) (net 17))
 (segment (start 132.45001 63.54999) (end 133.55401 63.54999) (width 0.5) (layer F.Cu) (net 17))
 (segment (start 129.5 66.5) (end 132.45001 63.54999) (width 0.5) (layer F.Cu) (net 17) (status 10))
 (segment (start 129.65576 85.12044) (end 130.03276 84.74344) (width 0.5) (layer B.Cu) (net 1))
 (segment (start 127.13776 85.12044) (end 129.65576 85.12044) (width 0.5) (layer B.Cu) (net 1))
 (segment (start 132.223 74.090002) (end 135.26516 77.132162) (width 0.5) (layer B.Cu) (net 1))
 (segment (start 132.223 73.66) (end 132.223 74.090002) (width 0.5) (layer B.Cu) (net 1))
 (segment (start 135.26516 77.132162) (end 135.26516 81.80324) (width 0.5) (layer B.Cu) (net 1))
 (segment (start 132.32496 84.74344) (end 130.03276 84.74344) (width 0.5) (layer B.Cu) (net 1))
 (segment (start 135.26516 81.80324) (end 132.32496 84.74344) (width 0.5) (layer B.Cu) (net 1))
 (segment (start 134.62 72.313) (end 134.223 72.71) (width 0.5) (layer B.Cu) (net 3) (status 30))
 (segment (start 134.62 70.896) (end 134.62 72.313) (width 0.5) (layer B.Cu) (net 3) (status 30)))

